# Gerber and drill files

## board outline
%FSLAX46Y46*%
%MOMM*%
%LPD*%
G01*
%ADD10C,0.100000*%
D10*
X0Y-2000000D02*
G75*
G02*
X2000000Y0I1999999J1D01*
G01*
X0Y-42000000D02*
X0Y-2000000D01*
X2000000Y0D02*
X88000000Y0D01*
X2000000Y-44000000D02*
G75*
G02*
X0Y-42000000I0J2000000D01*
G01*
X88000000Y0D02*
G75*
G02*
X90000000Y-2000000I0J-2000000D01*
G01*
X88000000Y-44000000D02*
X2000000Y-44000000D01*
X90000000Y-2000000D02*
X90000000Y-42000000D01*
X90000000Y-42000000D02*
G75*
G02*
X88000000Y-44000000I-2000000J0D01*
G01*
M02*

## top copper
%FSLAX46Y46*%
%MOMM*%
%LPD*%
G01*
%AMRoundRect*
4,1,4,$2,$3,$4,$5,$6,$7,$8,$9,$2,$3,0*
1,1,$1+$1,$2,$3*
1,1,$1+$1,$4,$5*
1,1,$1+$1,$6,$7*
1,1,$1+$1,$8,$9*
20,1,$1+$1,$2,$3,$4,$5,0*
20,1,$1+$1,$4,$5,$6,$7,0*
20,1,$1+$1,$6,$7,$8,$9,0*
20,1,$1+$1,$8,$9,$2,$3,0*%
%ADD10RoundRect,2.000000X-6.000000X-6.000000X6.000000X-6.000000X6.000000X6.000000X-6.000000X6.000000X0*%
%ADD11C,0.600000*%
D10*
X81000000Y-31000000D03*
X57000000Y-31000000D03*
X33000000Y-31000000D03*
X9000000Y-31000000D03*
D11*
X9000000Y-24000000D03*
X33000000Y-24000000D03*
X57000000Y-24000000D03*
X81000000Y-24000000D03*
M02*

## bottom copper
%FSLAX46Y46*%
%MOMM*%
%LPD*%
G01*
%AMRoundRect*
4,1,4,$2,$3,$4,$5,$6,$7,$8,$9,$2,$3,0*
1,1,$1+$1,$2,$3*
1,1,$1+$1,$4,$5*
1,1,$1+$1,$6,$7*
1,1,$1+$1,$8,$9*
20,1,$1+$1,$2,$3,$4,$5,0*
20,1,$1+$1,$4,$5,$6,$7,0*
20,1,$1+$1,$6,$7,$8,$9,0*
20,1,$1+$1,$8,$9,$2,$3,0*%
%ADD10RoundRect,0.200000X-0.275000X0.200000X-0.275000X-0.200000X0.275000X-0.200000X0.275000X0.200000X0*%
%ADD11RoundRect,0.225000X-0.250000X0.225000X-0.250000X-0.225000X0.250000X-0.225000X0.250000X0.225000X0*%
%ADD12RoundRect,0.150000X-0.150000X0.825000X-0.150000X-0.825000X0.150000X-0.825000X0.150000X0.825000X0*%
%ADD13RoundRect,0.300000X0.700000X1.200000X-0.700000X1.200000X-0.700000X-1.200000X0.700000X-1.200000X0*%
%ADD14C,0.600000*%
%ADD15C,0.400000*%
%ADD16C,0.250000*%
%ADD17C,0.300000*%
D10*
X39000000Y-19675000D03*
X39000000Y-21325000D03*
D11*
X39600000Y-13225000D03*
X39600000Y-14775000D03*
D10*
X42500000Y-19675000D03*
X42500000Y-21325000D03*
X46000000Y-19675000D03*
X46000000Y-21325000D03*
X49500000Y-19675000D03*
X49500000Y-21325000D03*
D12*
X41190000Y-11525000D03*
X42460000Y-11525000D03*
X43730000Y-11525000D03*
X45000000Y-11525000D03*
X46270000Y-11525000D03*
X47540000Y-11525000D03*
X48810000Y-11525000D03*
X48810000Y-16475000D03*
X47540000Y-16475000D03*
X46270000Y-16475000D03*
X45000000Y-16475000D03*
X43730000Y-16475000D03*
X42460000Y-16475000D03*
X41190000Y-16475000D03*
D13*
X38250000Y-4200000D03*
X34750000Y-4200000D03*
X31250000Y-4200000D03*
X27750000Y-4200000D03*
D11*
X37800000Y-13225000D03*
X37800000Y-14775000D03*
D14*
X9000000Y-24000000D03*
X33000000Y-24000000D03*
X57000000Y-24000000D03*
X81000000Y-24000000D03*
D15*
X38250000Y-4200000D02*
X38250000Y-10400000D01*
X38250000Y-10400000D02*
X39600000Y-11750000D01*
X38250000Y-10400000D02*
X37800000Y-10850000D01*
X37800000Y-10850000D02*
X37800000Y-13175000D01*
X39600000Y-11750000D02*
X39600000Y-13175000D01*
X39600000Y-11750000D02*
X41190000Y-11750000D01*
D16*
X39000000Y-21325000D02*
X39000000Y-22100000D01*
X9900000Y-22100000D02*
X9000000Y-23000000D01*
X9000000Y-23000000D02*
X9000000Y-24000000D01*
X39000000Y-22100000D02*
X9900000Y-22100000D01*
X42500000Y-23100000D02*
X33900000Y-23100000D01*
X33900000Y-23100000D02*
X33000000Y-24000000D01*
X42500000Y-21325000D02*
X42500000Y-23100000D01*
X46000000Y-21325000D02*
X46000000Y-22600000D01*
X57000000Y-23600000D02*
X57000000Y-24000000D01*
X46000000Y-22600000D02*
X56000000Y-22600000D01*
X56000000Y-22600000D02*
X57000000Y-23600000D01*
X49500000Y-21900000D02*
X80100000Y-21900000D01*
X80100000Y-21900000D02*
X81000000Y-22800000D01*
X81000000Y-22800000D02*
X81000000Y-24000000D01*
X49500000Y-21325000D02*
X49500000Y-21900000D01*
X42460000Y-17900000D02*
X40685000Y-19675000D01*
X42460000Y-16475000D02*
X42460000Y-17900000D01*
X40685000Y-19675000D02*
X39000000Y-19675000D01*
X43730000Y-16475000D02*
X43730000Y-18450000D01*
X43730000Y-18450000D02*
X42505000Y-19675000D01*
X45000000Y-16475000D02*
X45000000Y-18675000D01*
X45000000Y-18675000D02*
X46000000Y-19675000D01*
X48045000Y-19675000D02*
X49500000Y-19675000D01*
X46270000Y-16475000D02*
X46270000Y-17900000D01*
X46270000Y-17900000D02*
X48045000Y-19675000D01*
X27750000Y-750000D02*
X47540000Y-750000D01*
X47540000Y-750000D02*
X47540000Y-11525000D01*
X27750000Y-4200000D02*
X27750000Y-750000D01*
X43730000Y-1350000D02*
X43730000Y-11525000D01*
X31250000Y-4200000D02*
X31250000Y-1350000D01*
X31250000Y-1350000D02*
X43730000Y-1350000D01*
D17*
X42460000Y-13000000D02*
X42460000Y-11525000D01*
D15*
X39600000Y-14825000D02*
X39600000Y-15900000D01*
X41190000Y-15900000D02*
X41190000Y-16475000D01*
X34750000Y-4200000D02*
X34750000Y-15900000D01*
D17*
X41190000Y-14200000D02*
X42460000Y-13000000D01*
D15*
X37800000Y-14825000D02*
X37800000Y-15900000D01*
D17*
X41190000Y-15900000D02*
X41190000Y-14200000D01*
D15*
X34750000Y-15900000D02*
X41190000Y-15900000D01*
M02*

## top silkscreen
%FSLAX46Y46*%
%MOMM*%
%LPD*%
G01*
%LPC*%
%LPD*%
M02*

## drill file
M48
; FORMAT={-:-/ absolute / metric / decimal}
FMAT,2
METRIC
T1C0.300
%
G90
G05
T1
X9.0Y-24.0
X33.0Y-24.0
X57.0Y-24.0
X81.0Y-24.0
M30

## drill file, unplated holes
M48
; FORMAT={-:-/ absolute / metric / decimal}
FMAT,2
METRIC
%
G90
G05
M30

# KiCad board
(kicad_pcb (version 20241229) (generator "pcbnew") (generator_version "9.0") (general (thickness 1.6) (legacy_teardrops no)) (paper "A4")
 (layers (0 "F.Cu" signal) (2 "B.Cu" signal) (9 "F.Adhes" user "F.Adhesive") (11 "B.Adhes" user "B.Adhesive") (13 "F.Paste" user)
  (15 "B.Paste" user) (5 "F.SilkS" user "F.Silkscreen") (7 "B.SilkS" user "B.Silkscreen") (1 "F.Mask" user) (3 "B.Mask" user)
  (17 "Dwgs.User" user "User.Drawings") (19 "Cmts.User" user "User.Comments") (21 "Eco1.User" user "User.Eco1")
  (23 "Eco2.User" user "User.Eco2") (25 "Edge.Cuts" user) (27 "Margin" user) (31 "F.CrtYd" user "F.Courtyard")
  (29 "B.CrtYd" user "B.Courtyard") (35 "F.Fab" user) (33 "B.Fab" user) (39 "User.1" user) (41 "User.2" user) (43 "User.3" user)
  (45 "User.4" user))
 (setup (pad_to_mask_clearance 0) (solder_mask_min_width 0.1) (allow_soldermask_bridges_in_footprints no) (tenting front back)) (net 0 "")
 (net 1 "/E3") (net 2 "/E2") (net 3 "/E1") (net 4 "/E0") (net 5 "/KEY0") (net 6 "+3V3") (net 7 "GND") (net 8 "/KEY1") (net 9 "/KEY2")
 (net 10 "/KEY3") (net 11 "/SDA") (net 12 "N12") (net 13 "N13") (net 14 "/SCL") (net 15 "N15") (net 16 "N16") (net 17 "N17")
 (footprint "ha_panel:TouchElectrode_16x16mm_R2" (layer "F.Cu") (at 81 31)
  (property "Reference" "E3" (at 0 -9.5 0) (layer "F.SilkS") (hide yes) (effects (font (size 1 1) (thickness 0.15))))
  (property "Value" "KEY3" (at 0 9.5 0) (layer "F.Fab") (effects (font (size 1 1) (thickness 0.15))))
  (pad "1" smd roundrect (at 0 0) (size 16 16) (layers "F.Cu") (roundrect_rratio 0.125) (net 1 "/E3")))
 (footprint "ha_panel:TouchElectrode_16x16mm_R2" (layer "F.Cu") (at 57 31)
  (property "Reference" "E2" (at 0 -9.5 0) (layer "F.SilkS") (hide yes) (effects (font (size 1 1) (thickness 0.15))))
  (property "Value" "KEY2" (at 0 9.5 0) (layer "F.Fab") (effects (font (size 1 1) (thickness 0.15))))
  (pad "1" smd roundrect (at 0 0) (size 16 16) (layers "F.Cu") (roundrect_rratio 0.125) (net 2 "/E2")))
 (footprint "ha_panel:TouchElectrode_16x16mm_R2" (layer "F.Cu") (at 33 31)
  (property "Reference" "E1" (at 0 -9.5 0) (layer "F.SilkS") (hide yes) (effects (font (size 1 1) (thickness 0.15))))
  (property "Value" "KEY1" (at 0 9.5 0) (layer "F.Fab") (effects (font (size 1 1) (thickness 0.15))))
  (pad "1" smd roundrect (at 0 0) (size 16 16) (layers "F.Cu") (roundrect_rratio 0.125) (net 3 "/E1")))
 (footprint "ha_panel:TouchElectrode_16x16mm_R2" (layer "F.Cu") (at 9 31)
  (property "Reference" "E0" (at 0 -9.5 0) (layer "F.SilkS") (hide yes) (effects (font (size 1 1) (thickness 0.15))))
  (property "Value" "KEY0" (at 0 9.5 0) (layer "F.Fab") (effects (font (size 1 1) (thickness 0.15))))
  (pad "1" smd roundrect (at 0 0) (size 16 16) (layers "F.Cu") (roundrect_rratio 0.125) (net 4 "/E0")))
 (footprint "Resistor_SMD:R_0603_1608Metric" (layer "B.Cu") (at 39 20.5 -90)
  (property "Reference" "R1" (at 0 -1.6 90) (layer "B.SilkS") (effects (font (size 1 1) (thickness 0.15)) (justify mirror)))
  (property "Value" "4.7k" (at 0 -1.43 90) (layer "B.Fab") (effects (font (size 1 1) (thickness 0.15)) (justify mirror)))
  (pad "1" smd roundrect (at -0.825 0 270) (size 0.8 0.95) (layers "B.Cu" "B.Mask" "B.Paste") (roundrect_rratio 0.25) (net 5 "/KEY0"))
  (pad "2" smd roundrect (at 0.825 0 270) (size 0.8 0.95) (layers "B.Cu" "B.Mask" "B.Paste") (roundrect_rratio 0.25) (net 4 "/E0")))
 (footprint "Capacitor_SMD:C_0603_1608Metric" (layer "B.Cu") (at 39.6 14 -90)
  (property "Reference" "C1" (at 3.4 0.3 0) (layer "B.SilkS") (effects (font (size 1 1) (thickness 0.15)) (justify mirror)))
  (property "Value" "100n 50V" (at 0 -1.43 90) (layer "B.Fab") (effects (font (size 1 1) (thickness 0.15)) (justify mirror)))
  (pad "1" smd roundrect (at -0.775 0 270) (size 0.9 0.95) (layers "B.Cu" "B.Mask" "B.Paste") (roundrect_rratio 0.25) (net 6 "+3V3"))
  (pad "2" smd roundrect (at 0.775 0 270) (size 0.9 0.95) (layers "B.Cu" "B.Mask" "B.Paste") (roundrect_rratio 0.25) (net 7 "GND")))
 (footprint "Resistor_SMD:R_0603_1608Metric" (layer "B.Cu") (at 42.5 20.5 -90)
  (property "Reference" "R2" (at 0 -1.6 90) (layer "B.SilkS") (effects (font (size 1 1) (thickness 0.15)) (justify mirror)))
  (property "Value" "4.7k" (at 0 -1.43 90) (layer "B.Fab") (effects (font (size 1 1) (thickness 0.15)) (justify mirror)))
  (pad "1" smd roundrect (at -0.825 0 270) (size 0.8 0.95) (layers "B.Cu" "B.Mask" "B.Paste") (roundrect_rratio 0.25) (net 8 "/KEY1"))
  (pad "2" smd roundrect (at 0.825 0 270) (size 0.8 0.95) (layers "B.Cu" "B.Mask" "B.Paste") (roundrect_rratio 0.25) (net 3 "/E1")))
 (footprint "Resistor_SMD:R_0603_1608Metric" (layer "B.Cu") (at 46 20.5 -90)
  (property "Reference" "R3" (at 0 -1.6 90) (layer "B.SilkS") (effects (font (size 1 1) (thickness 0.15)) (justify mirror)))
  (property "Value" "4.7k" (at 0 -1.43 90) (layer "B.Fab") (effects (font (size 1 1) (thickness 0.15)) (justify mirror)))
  (pad "1" smd roundrect (at -0.825 0 270) (size 0.8 0.95) (layers "B.Cu" "B.Mask" "B.Paste") (roundrect_rratio 0.25) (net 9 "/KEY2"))
  (pad "2" smd roundrect (at 0.825 0 270) (size 0.8 0.95) (layers "B.Cu" "B.Mask" "B.Paste") (roundrect_rratio 0.25) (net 2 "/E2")))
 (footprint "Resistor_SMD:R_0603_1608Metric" (layer "B.Cu") (at 49.5 20.5 -90)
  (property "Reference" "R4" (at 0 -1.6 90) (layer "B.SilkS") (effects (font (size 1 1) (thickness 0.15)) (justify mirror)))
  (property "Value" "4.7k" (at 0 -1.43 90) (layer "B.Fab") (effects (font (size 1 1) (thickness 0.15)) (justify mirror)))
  (pad "1" smd roundrect (at -0.825 0 270) (size 0.8 0.95) (layers "B.Cu" "B.Mask" "B.Paste") (roundrect_rratio 0.25) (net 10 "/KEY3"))
  (pad "2" smd roundrect (at 0.825 0 270) (size 0.8 0.95) (layers "B.Cu" "B.Mask" "B.Paste") (roundrect_rratio 0.25) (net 1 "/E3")))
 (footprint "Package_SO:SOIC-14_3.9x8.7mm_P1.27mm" (layer "B.Cu") (at 45 14 -90)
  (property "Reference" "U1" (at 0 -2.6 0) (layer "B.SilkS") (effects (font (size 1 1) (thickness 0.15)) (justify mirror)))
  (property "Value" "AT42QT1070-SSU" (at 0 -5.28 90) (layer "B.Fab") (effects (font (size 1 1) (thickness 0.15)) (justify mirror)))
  (pad "1" smd roundrect (at -2.475 3.81 270) (size 1.95 0.6) (layers "B.Cu" "B.Mask" "B.Paste") (roundrect_rratio 0.25) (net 6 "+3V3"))
  (pad "2" smd roundrect (at -2.475 2.54 270) (size 1.95 0.6) (layers "B.Cu" "B.Mask" "B.Paste") (roundrect_rratio 0.25) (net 7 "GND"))
  (pad "3" smd roundrect (at -2.475 1.27 270) (size 1.95 0.6) (layers "B.Cu" "B.Mask" "B.Paste") (roundrect_rratio 0.25) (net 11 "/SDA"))
  (pad "4" smd roundrect (at -2.475 0 270) (size 1.95 0.6) (layers "B.Cu" "B.Mask" "B.Paste") (roundrect_rratio 0.25) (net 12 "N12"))
  (pad "5" smd roundrect (at -2.475 -1.27 270) (size 1.95 0.6) (layers "B.Cu" "B.Mask" "B.Paste") (roundrect_rratio 0.25) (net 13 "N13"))
  (pad "6" smd roundrect (at -2.475 -2.54 270) (size 1.95 0.6) (layers "B.Cu" "B.Mask" "B.Paste") (roundrect_rratio 0.25) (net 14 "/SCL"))
  (pad "7" smd roundrect (at -2.475 -3.81 270) (size 1.95 0.6) (layers "B.Cu" "B.Mask" "B.Paste") (roundrect_rratio 0.25) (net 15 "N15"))
  (pad "8" smd roundrect (at 2.475 -3.81 270) (size 1.95 0.6) (layers "B.Cu" "B.Mask" "B.Paste") (roundrect_rratio 0.25) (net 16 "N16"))
  (pad "9" smd roundrect (at 2.475 -2.54 270) (size 1.95 0.6) (layers "B.Cu" "B.Mask" "B.Paste") (roundrect_rratio 0.25) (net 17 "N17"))
  (pad "10" smd roundrect (at 2.475 -1.27 270) (size 1.95 0.6) (layers "B.Cu" "B.Mask" "B.Paste") (roundrect_rratio 0.25) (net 10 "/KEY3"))
  (pad "11" smd roundrect (at 2.475 0 270) (size 1.95 0.6) (layers "B.Cu" "B.Mask" "B.Paste") (roundrect_rratio 0.25) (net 9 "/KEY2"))
  (pad "12" smd roundrect (at 2.475 1.27 270) (size 1.95 0.6) (layers "B.Cu" "B.Mask" "B.Paste") (roundrect_rratio 0.25) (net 8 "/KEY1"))
  (pad "13" smd roundrect (at 2.475 2.54 270) (size 1.95 0.6) (layers "B.Cu" "B.Mask" "B.Paste") (roundrect_rratio 0.25) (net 5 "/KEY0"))
  (pad "14" smd roundrect (at 2.475 3.81 270) (size 1.95 0.6) (layers "B.Cu" "B.Mask" "B.Paste") (roundrect_rratio 0.25) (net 7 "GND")))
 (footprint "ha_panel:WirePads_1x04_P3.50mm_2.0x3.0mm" (layer "B.Cu") (at 38.25 4.2 180)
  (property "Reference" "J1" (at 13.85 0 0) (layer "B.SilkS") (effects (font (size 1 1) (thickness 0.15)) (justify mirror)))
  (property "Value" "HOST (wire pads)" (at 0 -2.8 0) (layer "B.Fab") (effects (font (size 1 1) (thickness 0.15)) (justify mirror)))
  (pad "1" smd roundrect (at 0 0 180) (size 2 3) (layers "B.Cu" "B.Mask") (roundrect_rratio 0.15) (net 6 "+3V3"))
  (pad "2" smd roundrect (at 3.5 0 180) (size 2 3) (layers "B.Cu" "B.Mask") (roundrect_rratio 0.15) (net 7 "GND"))
  (pad "3" smd roundrect (at 7 0 180) (size 2 3) (layers "B.Cu" "B.Mask") (roundrect_rratio 0.15) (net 11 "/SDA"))
  (pad "4" smd roundrect (at 10.5 0 180) (size 2 3) (layers "B.Cu" "B.Mask") (roundrect_rratio 0.15) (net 14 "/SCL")))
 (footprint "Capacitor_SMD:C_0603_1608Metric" (layer "B.Cu") (at 37.8 14 -90)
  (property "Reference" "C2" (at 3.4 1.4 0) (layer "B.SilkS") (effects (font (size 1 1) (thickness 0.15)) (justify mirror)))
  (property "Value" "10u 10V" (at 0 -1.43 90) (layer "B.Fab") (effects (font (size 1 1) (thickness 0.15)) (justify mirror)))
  (pad "1" smd roundrect (at -0.775 0 270) (size 0.9 0.95) (layers "B.Cu" "B.Mask" "B.Paste") (roundrect_rratio 0.25) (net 6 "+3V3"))
  (pad "2" smd roundrect (at 0.775 0 270) (size 0.9 0.95) (layers "B.Cu" "B.Mask" "B.Paste") (roundrect_rratio 0.25) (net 7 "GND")))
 (gr_arc (start 0 2) (mid 0.585786 0.585786) (end 2 0) (stroke (width 0.1) (type default)) (layer "Edge.Cuts"))
 (gr_line (start 0 42) (end 0 2) (stroke (width 0.1) (type default)) (layer "Edge.Cuts"))
 (gr_line (start 2 0) (end 88 0) (stroke (width 0.1) (type default)) (layer "Edge.Cuts"))
 (gr_arc (start 2 44) (mid 0.585786 43.414214) (end 0 42) (stroke (width 0.1) (type default)) (layer "Edge.Cuts"))
 (gr_arc (start 88 0) (mid 89.414214 0.585786) (end 90 2) (stroke (width 0.1) (type default)) (layer "Edge.Cuts"))
 (gr_line (start 88 44) (end 2 44) (stroke (width 0.1) (type default)) (layer "Edge.Cuts"))
 (gr_line (start 90 2) (end 90 42) (stroke (width 0.1) (type default)) (layer "Edge.Cuts"))
 (gr_arc (start 90 42) (mid 89.414214 43.414214) (end 88 44) (stroke (width 0.1) (type default)) (layer "Edge.Cuts"))
 (segment (start 38.25 4.2) (end 38.25 10.4) (width 0.4) (layer "B.Cu") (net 6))
 (segment (start 38.25 10.4) (end 39.6 11.75) (width 0.4) (layer "B.Cu") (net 6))
 (segment (start 38.25 10.4) (end 37.8 10.85) (width 0.4) (layer "B.Cu") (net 6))
 (segment (start 37.8 10.85) (end 37.8 13.175) (width 0.4) (layer "B.Cu") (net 6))
 (segment (start 39.6 11.75) (end 39.6 13.175) (width 0.4) (layer "B.Cu") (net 6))
 (segment (start 39.6 11.75) (end 41.19 11.75) (width 0.4) (layer "B.Cu") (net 6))
 (via (at 9 24) (size 0.6) (drill 0.3) (layers "F.Cu" "B.Cu") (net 4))
 (segment (start 39 21.325) (end 39 22.1) (width 0.25) (layer "B.Cu") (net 4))
 (segment (start 9.9 22.1) (end 9 23) (width 0.25) (layer "B.Cu") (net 4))
 (segment (start 9 23) (end 9 24) (width 0.25) (layer "B.Cu") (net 4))
 (segment (start 39 22.1) (end 9.9 22.1) (width 0.25) (layer "B.Cu") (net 4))
 (via (at 33 24) (size 0.6) (drill 0.3) (layers "F.Cu" "B.Cu") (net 3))
 (segment (start 42.5 23.1) (end 33.9 23.1) (width 0.25) (layer "B.Cu") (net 3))
 (segment (start 33.9 23.1) (end 33 24) (width 0.25) (layer "B.Cu") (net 3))
 (segment (start 42.5 21.325) (end 42.5 23.1) (width 0.25) (layer "B.Cu") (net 3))
 (via (at 57 24) (size 0.6) (drill 0.3) (layers "F.Cu" "B.Cu") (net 2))
 (segment (start 46 21.325) (end 46 22.6) (width 0.25) (layer "B.Cu") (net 2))
 (segment (start 57 23.6) (end 57 24) (width 0.25) (layer "B.Cu") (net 2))
 (segment (start 46 22.6) (end 56 22.6) (width 0.25) (layer "B.Cu") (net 2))
 (segment (start 56 22.6) (end 57 23.6) (width 0.25) (layer "B.Cu") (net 2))
 (via (at 81 24) (size 0.6) (drill 0.3) (layers "F.Cu" "B.Cu") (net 1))
 (segment (start 49.5 21.9) (end 80.1 21.9) (width 0.25) (layer "B.Cu") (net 1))
 (segment (start 80.1 21.9) (end 81 22.8) (width 0.25) (layer "B.Cu") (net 1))
 (segment (start 81 22.8) (end 81 24) (width 0.25) (layer "B.Cu") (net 1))
 (segment (start 49.5 21.325) (end 49.5 21.9) (width 0.25) (layer "B.Cu") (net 1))
 (segment (start 42.46 17.9) (end 40.685 19.675) (width 0.25) (layer "B.Cu") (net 5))
 (segment (start 42.46 16.475) (end 42.46 17.9) (width 0.25) (layer "B.Cu") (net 5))
 (segment (start 40.685 19.675) (end 39 19.675) (width 0.25) (layer "B.Cu") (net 5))
 (segment (start 43.73 16.475) (end 43.73 18.45) (width 0.25) (layer "B.Cu") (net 8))
 (segment (start 43.73 18.45) (end 42.505 19.675) (width 0.25) (layer "B.Cu") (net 8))
 (segment (start 45 16.475) (end 45 18.675) (width 0.25) (layer "B.Cu") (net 9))
 (segment (start 45 18.675) (end 46 19.675) (width 0.25) (layer "B.Cu") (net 9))
 (segment (start 48.045 19.675) (end 49.5 19.675) (width 0.25) (layer "B.Cu") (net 10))
 (segment (start 46.27 16.475) (end 46.27 17.9) (width 0.25) (layer "B.Cu") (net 10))
 (segment (start 46.27 17.9) (end 48.045 19.675) (width 0.25) (layer "B.Cu") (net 10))
 (segment (start 27.75 0.75) (end 47.54 0.75) (width 0.25) (layer "B.Cu") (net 14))
 (segment (start 47.54 0.75) (end 47.54 11.525) (width 0.25) (layer "B.Cu") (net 14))
 (segment (start 27.75 4.2) (end 27.75 0.75) (width 0.25) (layer "B.Cu") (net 14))
 (segment (start 43.73 1.35) (end 43.73 11.525) (width 0.25) (layer "B.Cu") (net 11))
 (segment (start 31.25 4.2) (end 31.25 1.35) (width 0.25) (layer "B.Cu") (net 11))
 (segment (start 31.25 1.35) (end 43.73 1.35) (width 0.25) (layer "B.Cu") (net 11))
 (segment (start 42.46 13) (end 42.46 11.525) (width 0.3) (layer "B.Cu") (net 7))
 (segment (start 39.6 14.825) (end 39.6 15.9) (width 0.4) (layer "B.Cu") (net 7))
 (segment (start 41.19 15.9) (end 41.19 16.475) (width 0.4) (layer "B.Cu") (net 7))
 (segment (start 34.75 4.2) (end 34.75 15.9) (width 0.4) (layer "B.Cu") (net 7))
 (segment (start 41.19 14.2) (end 42.46 13) (width 0.3) (layer "B.Cu") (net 7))
 (segment (start 37.8 14.825) (end 37.8 15.9) (width 0.4) (layer "B.Cu") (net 7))
 (segment (start 41.19 15.9) (end 41.19 14.2) (width 0.3) (layer "B.Cu") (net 7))
 (segment (start 34.75 15.9) (end 41.19 15.9) (width 0.4) (layer "B.Cu") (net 7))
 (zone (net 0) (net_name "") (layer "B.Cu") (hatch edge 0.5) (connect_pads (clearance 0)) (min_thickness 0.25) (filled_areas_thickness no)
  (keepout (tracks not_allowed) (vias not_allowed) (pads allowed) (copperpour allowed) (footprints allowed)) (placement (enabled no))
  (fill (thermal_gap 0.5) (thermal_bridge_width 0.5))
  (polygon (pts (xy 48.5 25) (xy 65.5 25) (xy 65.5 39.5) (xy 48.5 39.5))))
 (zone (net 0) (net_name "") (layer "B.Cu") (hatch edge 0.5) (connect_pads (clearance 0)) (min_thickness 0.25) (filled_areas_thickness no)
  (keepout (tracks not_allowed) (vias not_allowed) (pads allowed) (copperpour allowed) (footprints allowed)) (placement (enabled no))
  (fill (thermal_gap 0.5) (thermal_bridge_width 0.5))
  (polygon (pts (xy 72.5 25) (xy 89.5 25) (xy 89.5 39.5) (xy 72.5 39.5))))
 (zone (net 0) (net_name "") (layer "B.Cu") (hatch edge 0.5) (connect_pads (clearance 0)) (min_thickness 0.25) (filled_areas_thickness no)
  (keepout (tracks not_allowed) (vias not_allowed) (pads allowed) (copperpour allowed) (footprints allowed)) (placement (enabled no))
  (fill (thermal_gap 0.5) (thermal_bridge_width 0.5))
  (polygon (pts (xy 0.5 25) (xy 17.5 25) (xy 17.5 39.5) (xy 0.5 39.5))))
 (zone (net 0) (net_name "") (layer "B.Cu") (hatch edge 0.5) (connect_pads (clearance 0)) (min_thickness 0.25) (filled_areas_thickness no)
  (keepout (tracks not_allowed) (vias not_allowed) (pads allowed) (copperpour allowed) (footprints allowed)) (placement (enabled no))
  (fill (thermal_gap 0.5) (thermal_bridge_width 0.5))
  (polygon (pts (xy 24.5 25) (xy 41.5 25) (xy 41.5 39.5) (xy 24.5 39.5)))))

